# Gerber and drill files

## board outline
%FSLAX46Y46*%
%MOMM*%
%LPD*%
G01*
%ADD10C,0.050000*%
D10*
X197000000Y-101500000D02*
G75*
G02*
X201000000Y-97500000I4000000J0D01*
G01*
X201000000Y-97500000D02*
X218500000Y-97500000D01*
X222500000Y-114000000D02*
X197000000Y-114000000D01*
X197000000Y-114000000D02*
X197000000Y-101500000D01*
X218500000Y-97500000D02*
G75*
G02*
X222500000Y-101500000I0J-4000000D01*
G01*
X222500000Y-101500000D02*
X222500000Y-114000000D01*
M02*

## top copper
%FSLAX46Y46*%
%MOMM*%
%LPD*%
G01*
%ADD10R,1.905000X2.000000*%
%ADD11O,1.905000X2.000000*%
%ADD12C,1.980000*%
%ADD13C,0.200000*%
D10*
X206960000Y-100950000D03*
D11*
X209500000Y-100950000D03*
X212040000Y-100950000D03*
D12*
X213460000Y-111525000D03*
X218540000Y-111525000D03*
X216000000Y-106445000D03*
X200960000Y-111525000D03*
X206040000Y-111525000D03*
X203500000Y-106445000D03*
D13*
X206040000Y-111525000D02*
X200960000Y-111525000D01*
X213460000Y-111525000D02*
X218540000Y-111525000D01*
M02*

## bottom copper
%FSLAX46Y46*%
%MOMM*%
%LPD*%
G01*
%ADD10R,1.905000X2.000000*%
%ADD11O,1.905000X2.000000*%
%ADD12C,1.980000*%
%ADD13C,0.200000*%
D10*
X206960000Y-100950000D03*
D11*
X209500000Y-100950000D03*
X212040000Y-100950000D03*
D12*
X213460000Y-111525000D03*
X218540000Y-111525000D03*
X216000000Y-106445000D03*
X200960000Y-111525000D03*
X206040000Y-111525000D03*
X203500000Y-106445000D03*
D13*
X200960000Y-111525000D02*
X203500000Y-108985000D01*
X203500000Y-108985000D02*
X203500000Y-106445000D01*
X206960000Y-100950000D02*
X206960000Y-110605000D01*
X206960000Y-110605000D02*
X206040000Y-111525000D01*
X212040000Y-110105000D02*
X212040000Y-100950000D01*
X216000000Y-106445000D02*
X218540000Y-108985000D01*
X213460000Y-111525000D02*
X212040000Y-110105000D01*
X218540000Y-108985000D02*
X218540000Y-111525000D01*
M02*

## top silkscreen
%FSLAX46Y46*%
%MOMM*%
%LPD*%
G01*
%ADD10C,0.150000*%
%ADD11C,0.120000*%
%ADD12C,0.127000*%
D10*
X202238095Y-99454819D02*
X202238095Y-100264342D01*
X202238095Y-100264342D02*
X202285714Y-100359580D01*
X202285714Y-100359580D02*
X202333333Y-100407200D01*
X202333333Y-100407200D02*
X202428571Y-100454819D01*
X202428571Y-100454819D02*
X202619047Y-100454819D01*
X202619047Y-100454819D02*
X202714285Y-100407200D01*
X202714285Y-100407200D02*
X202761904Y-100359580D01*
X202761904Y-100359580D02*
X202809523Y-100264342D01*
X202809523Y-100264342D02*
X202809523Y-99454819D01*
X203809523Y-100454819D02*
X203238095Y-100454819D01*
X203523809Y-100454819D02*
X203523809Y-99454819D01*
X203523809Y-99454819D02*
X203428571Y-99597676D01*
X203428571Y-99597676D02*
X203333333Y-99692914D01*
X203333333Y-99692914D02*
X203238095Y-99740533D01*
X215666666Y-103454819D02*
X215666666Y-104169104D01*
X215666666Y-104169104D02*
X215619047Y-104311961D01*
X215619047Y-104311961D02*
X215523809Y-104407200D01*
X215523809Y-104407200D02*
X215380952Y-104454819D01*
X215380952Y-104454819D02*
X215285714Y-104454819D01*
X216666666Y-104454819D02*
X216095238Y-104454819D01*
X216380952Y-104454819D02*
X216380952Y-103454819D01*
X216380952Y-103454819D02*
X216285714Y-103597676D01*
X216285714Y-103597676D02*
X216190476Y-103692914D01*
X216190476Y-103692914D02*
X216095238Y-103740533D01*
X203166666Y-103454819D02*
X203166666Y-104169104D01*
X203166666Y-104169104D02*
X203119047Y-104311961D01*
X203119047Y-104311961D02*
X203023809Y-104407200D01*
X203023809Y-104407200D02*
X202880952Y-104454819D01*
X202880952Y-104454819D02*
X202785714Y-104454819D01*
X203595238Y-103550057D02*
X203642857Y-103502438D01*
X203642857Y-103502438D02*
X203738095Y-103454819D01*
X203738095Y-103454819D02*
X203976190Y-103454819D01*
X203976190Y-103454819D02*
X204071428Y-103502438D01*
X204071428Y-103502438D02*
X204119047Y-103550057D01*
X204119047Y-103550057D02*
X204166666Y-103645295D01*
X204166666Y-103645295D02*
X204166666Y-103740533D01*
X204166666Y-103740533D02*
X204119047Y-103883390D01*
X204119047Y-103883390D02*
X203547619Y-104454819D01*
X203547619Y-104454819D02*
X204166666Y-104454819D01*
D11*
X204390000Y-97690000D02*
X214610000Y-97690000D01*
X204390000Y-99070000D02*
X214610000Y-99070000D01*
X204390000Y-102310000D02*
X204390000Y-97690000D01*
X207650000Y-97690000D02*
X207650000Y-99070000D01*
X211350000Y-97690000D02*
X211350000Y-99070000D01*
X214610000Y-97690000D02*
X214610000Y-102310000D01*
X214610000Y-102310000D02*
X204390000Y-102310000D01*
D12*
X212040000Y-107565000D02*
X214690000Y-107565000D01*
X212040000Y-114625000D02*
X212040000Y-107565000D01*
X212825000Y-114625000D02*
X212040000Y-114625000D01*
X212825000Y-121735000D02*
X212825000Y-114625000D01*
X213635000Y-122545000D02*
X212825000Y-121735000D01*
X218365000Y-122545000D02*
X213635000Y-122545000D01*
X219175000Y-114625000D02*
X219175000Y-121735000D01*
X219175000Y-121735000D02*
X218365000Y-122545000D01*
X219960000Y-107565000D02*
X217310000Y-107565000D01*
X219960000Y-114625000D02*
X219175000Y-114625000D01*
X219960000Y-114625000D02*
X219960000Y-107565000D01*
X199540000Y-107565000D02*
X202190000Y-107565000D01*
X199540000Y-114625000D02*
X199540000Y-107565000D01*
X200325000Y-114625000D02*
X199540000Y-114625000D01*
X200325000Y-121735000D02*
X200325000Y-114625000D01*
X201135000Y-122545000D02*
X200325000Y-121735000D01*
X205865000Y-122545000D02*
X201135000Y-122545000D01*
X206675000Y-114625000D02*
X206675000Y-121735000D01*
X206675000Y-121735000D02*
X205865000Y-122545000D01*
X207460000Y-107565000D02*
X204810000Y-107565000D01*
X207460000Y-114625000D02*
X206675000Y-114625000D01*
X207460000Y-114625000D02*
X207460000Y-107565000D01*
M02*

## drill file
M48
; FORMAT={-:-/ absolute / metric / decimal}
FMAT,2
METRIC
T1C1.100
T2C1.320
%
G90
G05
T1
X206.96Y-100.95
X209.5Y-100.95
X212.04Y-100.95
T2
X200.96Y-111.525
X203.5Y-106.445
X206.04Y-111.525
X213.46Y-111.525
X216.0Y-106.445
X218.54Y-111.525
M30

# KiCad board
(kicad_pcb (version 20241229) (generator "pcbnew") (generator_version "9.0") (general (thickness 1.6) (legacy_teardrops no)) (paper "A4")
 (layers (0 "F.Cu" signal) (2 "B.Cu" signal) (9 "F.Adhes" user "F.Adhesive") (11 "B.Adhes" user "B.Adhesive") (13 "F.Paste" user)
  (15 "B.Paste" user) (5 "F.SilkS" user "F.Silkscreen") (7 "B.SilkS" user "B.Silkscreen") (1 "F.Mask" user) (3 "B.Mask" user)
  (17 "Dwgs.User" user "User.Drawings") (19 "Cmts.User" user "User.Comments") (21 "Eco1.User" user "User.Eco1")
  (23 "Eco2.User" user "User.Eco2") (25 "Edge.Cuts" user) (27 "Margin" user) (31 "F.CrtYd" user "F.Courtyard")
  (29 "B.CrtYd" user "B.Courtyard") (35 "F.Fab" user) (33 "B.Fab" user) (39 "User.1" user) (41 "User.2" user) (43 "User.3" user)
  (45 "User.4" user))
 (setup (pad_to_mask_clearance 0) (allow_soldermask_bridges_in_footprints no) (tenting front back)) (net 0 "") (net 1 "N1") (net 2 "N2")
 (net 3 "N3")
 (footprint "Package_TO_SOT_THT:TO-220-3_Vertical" (layer "F.Cu") (at 206.96 100.95)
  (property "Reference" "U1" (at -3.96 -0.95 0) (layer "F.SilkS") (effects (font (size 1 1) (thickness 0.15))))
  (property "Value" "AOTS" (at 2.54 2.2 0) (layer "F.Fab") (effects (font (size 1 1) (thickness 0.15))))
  (fp_line (start -2.57 -3.26) (end 7.65 -3.26) (stroke (width 0.12) (type solid)) (layer "F.SilkS"))
  (fp_line (start -2.57 -1.88) (end 7.65 -1.88) (stroke (width 0.12) (type solid)) (layer "F.SilkS"))
  (fp_line (start -2.57 1.36) (end -2.57 -3.26) (stroke (width 0.12) (type solid)) (layer "F.SilkS"))
  (fp_line (start 0.69 -3.26) (end 0.69 -1.88) (stroke (width 0.12) (type solid)) (layer "F.SilkS"))
  (fp_line (start 4.39 -3.26) (end 4.39 -1.88) (stroke (width 0.12) (type solid)) (layer "F.SilkS"))
  (fp_line (start 7.65 -3.26) (end 7.65 1.36) (stroke (width 0.12) (type solid)) (layer "F.SilkS"))
  (fp_line (start 7.65 1.36) (end -2.57 1.36) (stroke (width 0.12) (type solid)) (layer "F.SilkS"))
  (pad "1" thru_hole rect (at 0 0) (size 1.905 2) (drill 1.1) (layers "*.Cu" "*.Mask") (remove_unused_layers no) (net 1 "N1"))
  (pad "2" thru_hole oval (at 2.54 0) (size 1.905 2) (drill 1.1) (layers "*.Cu" "*.Mask") (remove_unused_layers no) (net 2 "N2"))
  (pad "3" thru_hole oval (at 5.08 0) (size 1.905 2) (drill 1.1) (layers "*.Cu" "*.Mask") (remove_unused_layers no) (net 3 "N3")))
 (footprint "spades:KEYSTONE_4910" (layer "F.Cu") (at 216 111.525 90)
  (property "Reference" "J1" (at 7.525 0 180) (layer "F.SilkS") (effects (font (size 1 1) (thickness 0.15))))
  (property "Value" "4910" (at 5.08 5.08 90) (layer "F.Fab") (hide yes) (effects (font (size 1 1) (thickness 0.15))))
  (fp_line (start 3.96 -3.96) (end 3.96 -1.31) (stroke (width 0.127) (type solid)) (layer "F.SilkS"))
  (fp_line (start -3.1 -3.96) (end 3.96 -3.96) (stroke (width 0.127) (type solid)) (layer "F.SilkS"))
  (fp_line (start -3.1 -3.175) (end -3.1 -3.96) (stroke (width 0.127) (type solid)) (layer "F.SilkS"))
  (fp_line (start -10.21 -3.175) (end -3.1 -3.175) (stroke (width 0.127) (type solid)) (layer "F.SilkS"))
  (fp_line (start -11.02 -2.365) (end -10.21 -3.175) (stroke (width 0.127) (type solid)) (layer "F.SilkS"))
  (fp_line (start -11.02 2.365) (end -11.02 -2.365) (stroke (width 0.127) (type solid)) (layer "F.SilkS"))
  (fp_line (start -3.1 3.175) (end -10.21 3.175) (stroke (width 0.127) (type solid)) (layer "F.SilkS"))
  (fp_line (start -10.21 3.175) (end -11.02 2.365) (stroke (width 0.127) (type solid)) (layer "F.SilkS"))
  (fp_line (start 3.96 3.96) (end 3.96 1.31) (stroke (width 0.127) (type solid)) (layer "F.SilkS"))
  (fp_line (start -3.1 3.96) (end -3.1 3.175) (stroke (width 0.127) (type solid)) (layer "F.SilkS"))
  (fp_line (start -3.1 3.96) (end 3.96 3.96) (stroke (width 0.127) (type solid)) (layer "F.SilkS"))
  (pad "1_1" thru_hole circle (at 0 -2.54 90) (size 1.98 1.98) (drill 1.32) (layers "*.Cu" "*.Mask") (remove_unused_layers no) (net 3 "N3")
   (solder_mask_margin 0.102))
  (pad "1_2" thru_hole circle (at 0 2.54 90) (size 1.98 1.98) (drill 1.32) (layers "*.Cu" "*.Mask") (remove_unused_layers no) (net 3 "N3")
   (solder_mask_margin 0.102))
  (pad "1_3" thru_hole circle (at 5.08 0 90) (size 1.98 1.98) (drill 1.32) (layers "*.Cu" "*.Mask") (remove_unused_layers no) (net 3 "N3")
   (solder_mask_margin 0.102)))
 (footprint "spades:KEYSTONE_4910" (layer "F.Cu") (at 203.5 111.525 90)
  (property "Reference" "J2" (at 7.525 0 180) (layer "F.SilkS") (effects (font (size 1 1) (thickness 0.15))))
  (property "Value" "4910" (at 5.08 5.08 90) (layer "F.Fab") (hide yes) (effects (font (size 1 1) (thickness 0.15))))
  (fp_line (start 3.96 -3.96) (end 3.96 -1.31) (stroke (width 0.127) (type solid)) (layer "F.SilkS"))
  (fp_line (start -3.1 -3.96) (end 3.96 -3.96) (stroke (width 0.127) (type solid)) (layer "F.SilkS"))
  (fp_line (start -3.1 -3.175) (end -3.1 -3.96) (stroke (width 0.127) (type solid)) (layer "F.SilkS"))
  (fp_line (start -10.21 -3.175) (end -3.1 -3.175) (stroke (width 0.127) (type solid)) (layer "F.SilkS"))
  (fp_line (start -11.02 -2.365) (end -10.21 -3.175) (stroke (width 0.127) (type solid)) (layer "F.SilkS"))
  (fp_line (start -11.02 2.365) (end -11.02 -2.365) (stroke (width 0.127) (type solid)) (layer "F.SilkS"))
  (fp_line (start -3.1 3.175) (end -10.21 3.175) (stroke (width 0.127) (type solid)) (layer "F.SilkS"))
  (fp_line (start -10.21 3.175) (end -11.02 2.365) (stroke (width 0.127) (type solid)) (layer "F.SilkS"))
  (fp_line (start 3.96 3.96) (end 3.96 1.31) (stroke (width 0.127) (type solid)) (layer "F.SilkS"))
  (fp_line (start -3.1 3.96) (end -3.1 3.175) (stroke (width 0.127) (type solid)) (layer "F.SilkS"))
  (fp_line (start -3.1 3.96) (end 3.96 3.96) (stroke (width 0.127) (type solid)) (layer "F.SilkS"))
  (pad "1_1" thru_hole circle (at 0 -2.54 90) (size 1.98 1.98) (drill 1.32) (layers "*.Cu" "*.Mask") (remove_unused_layers no) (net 1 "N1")
   (solder_mask_margin 0.102))
  (pad "1_2" thru_hole circle (at 0 2.54 90) (size 1.98 1.98) (drill 1.32) (layers "*.Cu" "*.Mask") (remove_unused_layers no) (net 1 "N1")
   (solder_mask_margin 0.102))
  (pad "1_3" thru_hole circle (at 5.08 0 90) (size 1.98 1.98) (drill 1.32) (layers "*.Cu" "*.Mask") (remove_unused_layers no) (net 1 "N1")
   (solder_mask_margin 0.102)))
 (gr_arc (start 197 101.5) (mid 198.171573 98.671573) (end 201 97.5) (stroke (width 0.05) (type default)) (layer "Edge.Cuts"))
 (gr_line (start 201 97.5) (end 218.5 97.5) (stroke (width 0.05) (type default)) (layer "Edge.Cuts"))
 (gr_line (start 222.5 114) (end 197 114) (stroke (width 0.05) (type default)) (layer "Edge.Cuts"))
 (gr_line (start 197 114) (end 197 101.5) (stroke (width 0.05) (type default)) (layer "Edge.Cuts"))
 (gr_arc (start 218.5 97.5) (mid 221.328427 98.671573) (end 222.5 101.5) (stroke (width 0.05) (type default)) (layer "Edge.Cuts"))
 (gr_line (start 222.5 101.5) (end 222.5 114) (stroke (width 0.05) (type default)) (layer "Edge.Cuts"))
 (segment (start 206.04 111.525) (end 200.96 111.525) (width 0.2) (layer "F.Cu") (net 1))
 (segment (start 200.96 111.525) (end 203.5 108.985) (width 0.2) (layer "B.Cu") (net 1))
 (segment (start 203.5 108.985) (end 203.5 106.445) (width 0.2) (layer "B.Cu") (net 1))
 (segment (start 206.96 100.95) (end 206.96 110.605) (width 0.2) (layer "B.Cu") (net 1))
 (segment (start 206.96 110.605) (end 206.04 111.525) (width 0.2) (layer "B.Cu") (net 1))
 (segment (start 213.46 111.525) (end 218.54 111.525) (width 0.2) (layer "F.Cu") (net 3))
 (segment (start 212.04 110.105) (end 212.04 100.95) (width 0.2) (layer "B.Cu") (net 3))
 (segment (start 216 106.445) (end 218.54 108.985) (width 0.2) (layer "B.Cu") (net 3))
 (segment (start 213.46 111.525) (end 212.04 110.105) (width 0.2) (layer "B.Cu") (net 3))
 (segment (start 218.54 108.985) (end 218.54 111.525) (width 0.2) (layer "B.Cu") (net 3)))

